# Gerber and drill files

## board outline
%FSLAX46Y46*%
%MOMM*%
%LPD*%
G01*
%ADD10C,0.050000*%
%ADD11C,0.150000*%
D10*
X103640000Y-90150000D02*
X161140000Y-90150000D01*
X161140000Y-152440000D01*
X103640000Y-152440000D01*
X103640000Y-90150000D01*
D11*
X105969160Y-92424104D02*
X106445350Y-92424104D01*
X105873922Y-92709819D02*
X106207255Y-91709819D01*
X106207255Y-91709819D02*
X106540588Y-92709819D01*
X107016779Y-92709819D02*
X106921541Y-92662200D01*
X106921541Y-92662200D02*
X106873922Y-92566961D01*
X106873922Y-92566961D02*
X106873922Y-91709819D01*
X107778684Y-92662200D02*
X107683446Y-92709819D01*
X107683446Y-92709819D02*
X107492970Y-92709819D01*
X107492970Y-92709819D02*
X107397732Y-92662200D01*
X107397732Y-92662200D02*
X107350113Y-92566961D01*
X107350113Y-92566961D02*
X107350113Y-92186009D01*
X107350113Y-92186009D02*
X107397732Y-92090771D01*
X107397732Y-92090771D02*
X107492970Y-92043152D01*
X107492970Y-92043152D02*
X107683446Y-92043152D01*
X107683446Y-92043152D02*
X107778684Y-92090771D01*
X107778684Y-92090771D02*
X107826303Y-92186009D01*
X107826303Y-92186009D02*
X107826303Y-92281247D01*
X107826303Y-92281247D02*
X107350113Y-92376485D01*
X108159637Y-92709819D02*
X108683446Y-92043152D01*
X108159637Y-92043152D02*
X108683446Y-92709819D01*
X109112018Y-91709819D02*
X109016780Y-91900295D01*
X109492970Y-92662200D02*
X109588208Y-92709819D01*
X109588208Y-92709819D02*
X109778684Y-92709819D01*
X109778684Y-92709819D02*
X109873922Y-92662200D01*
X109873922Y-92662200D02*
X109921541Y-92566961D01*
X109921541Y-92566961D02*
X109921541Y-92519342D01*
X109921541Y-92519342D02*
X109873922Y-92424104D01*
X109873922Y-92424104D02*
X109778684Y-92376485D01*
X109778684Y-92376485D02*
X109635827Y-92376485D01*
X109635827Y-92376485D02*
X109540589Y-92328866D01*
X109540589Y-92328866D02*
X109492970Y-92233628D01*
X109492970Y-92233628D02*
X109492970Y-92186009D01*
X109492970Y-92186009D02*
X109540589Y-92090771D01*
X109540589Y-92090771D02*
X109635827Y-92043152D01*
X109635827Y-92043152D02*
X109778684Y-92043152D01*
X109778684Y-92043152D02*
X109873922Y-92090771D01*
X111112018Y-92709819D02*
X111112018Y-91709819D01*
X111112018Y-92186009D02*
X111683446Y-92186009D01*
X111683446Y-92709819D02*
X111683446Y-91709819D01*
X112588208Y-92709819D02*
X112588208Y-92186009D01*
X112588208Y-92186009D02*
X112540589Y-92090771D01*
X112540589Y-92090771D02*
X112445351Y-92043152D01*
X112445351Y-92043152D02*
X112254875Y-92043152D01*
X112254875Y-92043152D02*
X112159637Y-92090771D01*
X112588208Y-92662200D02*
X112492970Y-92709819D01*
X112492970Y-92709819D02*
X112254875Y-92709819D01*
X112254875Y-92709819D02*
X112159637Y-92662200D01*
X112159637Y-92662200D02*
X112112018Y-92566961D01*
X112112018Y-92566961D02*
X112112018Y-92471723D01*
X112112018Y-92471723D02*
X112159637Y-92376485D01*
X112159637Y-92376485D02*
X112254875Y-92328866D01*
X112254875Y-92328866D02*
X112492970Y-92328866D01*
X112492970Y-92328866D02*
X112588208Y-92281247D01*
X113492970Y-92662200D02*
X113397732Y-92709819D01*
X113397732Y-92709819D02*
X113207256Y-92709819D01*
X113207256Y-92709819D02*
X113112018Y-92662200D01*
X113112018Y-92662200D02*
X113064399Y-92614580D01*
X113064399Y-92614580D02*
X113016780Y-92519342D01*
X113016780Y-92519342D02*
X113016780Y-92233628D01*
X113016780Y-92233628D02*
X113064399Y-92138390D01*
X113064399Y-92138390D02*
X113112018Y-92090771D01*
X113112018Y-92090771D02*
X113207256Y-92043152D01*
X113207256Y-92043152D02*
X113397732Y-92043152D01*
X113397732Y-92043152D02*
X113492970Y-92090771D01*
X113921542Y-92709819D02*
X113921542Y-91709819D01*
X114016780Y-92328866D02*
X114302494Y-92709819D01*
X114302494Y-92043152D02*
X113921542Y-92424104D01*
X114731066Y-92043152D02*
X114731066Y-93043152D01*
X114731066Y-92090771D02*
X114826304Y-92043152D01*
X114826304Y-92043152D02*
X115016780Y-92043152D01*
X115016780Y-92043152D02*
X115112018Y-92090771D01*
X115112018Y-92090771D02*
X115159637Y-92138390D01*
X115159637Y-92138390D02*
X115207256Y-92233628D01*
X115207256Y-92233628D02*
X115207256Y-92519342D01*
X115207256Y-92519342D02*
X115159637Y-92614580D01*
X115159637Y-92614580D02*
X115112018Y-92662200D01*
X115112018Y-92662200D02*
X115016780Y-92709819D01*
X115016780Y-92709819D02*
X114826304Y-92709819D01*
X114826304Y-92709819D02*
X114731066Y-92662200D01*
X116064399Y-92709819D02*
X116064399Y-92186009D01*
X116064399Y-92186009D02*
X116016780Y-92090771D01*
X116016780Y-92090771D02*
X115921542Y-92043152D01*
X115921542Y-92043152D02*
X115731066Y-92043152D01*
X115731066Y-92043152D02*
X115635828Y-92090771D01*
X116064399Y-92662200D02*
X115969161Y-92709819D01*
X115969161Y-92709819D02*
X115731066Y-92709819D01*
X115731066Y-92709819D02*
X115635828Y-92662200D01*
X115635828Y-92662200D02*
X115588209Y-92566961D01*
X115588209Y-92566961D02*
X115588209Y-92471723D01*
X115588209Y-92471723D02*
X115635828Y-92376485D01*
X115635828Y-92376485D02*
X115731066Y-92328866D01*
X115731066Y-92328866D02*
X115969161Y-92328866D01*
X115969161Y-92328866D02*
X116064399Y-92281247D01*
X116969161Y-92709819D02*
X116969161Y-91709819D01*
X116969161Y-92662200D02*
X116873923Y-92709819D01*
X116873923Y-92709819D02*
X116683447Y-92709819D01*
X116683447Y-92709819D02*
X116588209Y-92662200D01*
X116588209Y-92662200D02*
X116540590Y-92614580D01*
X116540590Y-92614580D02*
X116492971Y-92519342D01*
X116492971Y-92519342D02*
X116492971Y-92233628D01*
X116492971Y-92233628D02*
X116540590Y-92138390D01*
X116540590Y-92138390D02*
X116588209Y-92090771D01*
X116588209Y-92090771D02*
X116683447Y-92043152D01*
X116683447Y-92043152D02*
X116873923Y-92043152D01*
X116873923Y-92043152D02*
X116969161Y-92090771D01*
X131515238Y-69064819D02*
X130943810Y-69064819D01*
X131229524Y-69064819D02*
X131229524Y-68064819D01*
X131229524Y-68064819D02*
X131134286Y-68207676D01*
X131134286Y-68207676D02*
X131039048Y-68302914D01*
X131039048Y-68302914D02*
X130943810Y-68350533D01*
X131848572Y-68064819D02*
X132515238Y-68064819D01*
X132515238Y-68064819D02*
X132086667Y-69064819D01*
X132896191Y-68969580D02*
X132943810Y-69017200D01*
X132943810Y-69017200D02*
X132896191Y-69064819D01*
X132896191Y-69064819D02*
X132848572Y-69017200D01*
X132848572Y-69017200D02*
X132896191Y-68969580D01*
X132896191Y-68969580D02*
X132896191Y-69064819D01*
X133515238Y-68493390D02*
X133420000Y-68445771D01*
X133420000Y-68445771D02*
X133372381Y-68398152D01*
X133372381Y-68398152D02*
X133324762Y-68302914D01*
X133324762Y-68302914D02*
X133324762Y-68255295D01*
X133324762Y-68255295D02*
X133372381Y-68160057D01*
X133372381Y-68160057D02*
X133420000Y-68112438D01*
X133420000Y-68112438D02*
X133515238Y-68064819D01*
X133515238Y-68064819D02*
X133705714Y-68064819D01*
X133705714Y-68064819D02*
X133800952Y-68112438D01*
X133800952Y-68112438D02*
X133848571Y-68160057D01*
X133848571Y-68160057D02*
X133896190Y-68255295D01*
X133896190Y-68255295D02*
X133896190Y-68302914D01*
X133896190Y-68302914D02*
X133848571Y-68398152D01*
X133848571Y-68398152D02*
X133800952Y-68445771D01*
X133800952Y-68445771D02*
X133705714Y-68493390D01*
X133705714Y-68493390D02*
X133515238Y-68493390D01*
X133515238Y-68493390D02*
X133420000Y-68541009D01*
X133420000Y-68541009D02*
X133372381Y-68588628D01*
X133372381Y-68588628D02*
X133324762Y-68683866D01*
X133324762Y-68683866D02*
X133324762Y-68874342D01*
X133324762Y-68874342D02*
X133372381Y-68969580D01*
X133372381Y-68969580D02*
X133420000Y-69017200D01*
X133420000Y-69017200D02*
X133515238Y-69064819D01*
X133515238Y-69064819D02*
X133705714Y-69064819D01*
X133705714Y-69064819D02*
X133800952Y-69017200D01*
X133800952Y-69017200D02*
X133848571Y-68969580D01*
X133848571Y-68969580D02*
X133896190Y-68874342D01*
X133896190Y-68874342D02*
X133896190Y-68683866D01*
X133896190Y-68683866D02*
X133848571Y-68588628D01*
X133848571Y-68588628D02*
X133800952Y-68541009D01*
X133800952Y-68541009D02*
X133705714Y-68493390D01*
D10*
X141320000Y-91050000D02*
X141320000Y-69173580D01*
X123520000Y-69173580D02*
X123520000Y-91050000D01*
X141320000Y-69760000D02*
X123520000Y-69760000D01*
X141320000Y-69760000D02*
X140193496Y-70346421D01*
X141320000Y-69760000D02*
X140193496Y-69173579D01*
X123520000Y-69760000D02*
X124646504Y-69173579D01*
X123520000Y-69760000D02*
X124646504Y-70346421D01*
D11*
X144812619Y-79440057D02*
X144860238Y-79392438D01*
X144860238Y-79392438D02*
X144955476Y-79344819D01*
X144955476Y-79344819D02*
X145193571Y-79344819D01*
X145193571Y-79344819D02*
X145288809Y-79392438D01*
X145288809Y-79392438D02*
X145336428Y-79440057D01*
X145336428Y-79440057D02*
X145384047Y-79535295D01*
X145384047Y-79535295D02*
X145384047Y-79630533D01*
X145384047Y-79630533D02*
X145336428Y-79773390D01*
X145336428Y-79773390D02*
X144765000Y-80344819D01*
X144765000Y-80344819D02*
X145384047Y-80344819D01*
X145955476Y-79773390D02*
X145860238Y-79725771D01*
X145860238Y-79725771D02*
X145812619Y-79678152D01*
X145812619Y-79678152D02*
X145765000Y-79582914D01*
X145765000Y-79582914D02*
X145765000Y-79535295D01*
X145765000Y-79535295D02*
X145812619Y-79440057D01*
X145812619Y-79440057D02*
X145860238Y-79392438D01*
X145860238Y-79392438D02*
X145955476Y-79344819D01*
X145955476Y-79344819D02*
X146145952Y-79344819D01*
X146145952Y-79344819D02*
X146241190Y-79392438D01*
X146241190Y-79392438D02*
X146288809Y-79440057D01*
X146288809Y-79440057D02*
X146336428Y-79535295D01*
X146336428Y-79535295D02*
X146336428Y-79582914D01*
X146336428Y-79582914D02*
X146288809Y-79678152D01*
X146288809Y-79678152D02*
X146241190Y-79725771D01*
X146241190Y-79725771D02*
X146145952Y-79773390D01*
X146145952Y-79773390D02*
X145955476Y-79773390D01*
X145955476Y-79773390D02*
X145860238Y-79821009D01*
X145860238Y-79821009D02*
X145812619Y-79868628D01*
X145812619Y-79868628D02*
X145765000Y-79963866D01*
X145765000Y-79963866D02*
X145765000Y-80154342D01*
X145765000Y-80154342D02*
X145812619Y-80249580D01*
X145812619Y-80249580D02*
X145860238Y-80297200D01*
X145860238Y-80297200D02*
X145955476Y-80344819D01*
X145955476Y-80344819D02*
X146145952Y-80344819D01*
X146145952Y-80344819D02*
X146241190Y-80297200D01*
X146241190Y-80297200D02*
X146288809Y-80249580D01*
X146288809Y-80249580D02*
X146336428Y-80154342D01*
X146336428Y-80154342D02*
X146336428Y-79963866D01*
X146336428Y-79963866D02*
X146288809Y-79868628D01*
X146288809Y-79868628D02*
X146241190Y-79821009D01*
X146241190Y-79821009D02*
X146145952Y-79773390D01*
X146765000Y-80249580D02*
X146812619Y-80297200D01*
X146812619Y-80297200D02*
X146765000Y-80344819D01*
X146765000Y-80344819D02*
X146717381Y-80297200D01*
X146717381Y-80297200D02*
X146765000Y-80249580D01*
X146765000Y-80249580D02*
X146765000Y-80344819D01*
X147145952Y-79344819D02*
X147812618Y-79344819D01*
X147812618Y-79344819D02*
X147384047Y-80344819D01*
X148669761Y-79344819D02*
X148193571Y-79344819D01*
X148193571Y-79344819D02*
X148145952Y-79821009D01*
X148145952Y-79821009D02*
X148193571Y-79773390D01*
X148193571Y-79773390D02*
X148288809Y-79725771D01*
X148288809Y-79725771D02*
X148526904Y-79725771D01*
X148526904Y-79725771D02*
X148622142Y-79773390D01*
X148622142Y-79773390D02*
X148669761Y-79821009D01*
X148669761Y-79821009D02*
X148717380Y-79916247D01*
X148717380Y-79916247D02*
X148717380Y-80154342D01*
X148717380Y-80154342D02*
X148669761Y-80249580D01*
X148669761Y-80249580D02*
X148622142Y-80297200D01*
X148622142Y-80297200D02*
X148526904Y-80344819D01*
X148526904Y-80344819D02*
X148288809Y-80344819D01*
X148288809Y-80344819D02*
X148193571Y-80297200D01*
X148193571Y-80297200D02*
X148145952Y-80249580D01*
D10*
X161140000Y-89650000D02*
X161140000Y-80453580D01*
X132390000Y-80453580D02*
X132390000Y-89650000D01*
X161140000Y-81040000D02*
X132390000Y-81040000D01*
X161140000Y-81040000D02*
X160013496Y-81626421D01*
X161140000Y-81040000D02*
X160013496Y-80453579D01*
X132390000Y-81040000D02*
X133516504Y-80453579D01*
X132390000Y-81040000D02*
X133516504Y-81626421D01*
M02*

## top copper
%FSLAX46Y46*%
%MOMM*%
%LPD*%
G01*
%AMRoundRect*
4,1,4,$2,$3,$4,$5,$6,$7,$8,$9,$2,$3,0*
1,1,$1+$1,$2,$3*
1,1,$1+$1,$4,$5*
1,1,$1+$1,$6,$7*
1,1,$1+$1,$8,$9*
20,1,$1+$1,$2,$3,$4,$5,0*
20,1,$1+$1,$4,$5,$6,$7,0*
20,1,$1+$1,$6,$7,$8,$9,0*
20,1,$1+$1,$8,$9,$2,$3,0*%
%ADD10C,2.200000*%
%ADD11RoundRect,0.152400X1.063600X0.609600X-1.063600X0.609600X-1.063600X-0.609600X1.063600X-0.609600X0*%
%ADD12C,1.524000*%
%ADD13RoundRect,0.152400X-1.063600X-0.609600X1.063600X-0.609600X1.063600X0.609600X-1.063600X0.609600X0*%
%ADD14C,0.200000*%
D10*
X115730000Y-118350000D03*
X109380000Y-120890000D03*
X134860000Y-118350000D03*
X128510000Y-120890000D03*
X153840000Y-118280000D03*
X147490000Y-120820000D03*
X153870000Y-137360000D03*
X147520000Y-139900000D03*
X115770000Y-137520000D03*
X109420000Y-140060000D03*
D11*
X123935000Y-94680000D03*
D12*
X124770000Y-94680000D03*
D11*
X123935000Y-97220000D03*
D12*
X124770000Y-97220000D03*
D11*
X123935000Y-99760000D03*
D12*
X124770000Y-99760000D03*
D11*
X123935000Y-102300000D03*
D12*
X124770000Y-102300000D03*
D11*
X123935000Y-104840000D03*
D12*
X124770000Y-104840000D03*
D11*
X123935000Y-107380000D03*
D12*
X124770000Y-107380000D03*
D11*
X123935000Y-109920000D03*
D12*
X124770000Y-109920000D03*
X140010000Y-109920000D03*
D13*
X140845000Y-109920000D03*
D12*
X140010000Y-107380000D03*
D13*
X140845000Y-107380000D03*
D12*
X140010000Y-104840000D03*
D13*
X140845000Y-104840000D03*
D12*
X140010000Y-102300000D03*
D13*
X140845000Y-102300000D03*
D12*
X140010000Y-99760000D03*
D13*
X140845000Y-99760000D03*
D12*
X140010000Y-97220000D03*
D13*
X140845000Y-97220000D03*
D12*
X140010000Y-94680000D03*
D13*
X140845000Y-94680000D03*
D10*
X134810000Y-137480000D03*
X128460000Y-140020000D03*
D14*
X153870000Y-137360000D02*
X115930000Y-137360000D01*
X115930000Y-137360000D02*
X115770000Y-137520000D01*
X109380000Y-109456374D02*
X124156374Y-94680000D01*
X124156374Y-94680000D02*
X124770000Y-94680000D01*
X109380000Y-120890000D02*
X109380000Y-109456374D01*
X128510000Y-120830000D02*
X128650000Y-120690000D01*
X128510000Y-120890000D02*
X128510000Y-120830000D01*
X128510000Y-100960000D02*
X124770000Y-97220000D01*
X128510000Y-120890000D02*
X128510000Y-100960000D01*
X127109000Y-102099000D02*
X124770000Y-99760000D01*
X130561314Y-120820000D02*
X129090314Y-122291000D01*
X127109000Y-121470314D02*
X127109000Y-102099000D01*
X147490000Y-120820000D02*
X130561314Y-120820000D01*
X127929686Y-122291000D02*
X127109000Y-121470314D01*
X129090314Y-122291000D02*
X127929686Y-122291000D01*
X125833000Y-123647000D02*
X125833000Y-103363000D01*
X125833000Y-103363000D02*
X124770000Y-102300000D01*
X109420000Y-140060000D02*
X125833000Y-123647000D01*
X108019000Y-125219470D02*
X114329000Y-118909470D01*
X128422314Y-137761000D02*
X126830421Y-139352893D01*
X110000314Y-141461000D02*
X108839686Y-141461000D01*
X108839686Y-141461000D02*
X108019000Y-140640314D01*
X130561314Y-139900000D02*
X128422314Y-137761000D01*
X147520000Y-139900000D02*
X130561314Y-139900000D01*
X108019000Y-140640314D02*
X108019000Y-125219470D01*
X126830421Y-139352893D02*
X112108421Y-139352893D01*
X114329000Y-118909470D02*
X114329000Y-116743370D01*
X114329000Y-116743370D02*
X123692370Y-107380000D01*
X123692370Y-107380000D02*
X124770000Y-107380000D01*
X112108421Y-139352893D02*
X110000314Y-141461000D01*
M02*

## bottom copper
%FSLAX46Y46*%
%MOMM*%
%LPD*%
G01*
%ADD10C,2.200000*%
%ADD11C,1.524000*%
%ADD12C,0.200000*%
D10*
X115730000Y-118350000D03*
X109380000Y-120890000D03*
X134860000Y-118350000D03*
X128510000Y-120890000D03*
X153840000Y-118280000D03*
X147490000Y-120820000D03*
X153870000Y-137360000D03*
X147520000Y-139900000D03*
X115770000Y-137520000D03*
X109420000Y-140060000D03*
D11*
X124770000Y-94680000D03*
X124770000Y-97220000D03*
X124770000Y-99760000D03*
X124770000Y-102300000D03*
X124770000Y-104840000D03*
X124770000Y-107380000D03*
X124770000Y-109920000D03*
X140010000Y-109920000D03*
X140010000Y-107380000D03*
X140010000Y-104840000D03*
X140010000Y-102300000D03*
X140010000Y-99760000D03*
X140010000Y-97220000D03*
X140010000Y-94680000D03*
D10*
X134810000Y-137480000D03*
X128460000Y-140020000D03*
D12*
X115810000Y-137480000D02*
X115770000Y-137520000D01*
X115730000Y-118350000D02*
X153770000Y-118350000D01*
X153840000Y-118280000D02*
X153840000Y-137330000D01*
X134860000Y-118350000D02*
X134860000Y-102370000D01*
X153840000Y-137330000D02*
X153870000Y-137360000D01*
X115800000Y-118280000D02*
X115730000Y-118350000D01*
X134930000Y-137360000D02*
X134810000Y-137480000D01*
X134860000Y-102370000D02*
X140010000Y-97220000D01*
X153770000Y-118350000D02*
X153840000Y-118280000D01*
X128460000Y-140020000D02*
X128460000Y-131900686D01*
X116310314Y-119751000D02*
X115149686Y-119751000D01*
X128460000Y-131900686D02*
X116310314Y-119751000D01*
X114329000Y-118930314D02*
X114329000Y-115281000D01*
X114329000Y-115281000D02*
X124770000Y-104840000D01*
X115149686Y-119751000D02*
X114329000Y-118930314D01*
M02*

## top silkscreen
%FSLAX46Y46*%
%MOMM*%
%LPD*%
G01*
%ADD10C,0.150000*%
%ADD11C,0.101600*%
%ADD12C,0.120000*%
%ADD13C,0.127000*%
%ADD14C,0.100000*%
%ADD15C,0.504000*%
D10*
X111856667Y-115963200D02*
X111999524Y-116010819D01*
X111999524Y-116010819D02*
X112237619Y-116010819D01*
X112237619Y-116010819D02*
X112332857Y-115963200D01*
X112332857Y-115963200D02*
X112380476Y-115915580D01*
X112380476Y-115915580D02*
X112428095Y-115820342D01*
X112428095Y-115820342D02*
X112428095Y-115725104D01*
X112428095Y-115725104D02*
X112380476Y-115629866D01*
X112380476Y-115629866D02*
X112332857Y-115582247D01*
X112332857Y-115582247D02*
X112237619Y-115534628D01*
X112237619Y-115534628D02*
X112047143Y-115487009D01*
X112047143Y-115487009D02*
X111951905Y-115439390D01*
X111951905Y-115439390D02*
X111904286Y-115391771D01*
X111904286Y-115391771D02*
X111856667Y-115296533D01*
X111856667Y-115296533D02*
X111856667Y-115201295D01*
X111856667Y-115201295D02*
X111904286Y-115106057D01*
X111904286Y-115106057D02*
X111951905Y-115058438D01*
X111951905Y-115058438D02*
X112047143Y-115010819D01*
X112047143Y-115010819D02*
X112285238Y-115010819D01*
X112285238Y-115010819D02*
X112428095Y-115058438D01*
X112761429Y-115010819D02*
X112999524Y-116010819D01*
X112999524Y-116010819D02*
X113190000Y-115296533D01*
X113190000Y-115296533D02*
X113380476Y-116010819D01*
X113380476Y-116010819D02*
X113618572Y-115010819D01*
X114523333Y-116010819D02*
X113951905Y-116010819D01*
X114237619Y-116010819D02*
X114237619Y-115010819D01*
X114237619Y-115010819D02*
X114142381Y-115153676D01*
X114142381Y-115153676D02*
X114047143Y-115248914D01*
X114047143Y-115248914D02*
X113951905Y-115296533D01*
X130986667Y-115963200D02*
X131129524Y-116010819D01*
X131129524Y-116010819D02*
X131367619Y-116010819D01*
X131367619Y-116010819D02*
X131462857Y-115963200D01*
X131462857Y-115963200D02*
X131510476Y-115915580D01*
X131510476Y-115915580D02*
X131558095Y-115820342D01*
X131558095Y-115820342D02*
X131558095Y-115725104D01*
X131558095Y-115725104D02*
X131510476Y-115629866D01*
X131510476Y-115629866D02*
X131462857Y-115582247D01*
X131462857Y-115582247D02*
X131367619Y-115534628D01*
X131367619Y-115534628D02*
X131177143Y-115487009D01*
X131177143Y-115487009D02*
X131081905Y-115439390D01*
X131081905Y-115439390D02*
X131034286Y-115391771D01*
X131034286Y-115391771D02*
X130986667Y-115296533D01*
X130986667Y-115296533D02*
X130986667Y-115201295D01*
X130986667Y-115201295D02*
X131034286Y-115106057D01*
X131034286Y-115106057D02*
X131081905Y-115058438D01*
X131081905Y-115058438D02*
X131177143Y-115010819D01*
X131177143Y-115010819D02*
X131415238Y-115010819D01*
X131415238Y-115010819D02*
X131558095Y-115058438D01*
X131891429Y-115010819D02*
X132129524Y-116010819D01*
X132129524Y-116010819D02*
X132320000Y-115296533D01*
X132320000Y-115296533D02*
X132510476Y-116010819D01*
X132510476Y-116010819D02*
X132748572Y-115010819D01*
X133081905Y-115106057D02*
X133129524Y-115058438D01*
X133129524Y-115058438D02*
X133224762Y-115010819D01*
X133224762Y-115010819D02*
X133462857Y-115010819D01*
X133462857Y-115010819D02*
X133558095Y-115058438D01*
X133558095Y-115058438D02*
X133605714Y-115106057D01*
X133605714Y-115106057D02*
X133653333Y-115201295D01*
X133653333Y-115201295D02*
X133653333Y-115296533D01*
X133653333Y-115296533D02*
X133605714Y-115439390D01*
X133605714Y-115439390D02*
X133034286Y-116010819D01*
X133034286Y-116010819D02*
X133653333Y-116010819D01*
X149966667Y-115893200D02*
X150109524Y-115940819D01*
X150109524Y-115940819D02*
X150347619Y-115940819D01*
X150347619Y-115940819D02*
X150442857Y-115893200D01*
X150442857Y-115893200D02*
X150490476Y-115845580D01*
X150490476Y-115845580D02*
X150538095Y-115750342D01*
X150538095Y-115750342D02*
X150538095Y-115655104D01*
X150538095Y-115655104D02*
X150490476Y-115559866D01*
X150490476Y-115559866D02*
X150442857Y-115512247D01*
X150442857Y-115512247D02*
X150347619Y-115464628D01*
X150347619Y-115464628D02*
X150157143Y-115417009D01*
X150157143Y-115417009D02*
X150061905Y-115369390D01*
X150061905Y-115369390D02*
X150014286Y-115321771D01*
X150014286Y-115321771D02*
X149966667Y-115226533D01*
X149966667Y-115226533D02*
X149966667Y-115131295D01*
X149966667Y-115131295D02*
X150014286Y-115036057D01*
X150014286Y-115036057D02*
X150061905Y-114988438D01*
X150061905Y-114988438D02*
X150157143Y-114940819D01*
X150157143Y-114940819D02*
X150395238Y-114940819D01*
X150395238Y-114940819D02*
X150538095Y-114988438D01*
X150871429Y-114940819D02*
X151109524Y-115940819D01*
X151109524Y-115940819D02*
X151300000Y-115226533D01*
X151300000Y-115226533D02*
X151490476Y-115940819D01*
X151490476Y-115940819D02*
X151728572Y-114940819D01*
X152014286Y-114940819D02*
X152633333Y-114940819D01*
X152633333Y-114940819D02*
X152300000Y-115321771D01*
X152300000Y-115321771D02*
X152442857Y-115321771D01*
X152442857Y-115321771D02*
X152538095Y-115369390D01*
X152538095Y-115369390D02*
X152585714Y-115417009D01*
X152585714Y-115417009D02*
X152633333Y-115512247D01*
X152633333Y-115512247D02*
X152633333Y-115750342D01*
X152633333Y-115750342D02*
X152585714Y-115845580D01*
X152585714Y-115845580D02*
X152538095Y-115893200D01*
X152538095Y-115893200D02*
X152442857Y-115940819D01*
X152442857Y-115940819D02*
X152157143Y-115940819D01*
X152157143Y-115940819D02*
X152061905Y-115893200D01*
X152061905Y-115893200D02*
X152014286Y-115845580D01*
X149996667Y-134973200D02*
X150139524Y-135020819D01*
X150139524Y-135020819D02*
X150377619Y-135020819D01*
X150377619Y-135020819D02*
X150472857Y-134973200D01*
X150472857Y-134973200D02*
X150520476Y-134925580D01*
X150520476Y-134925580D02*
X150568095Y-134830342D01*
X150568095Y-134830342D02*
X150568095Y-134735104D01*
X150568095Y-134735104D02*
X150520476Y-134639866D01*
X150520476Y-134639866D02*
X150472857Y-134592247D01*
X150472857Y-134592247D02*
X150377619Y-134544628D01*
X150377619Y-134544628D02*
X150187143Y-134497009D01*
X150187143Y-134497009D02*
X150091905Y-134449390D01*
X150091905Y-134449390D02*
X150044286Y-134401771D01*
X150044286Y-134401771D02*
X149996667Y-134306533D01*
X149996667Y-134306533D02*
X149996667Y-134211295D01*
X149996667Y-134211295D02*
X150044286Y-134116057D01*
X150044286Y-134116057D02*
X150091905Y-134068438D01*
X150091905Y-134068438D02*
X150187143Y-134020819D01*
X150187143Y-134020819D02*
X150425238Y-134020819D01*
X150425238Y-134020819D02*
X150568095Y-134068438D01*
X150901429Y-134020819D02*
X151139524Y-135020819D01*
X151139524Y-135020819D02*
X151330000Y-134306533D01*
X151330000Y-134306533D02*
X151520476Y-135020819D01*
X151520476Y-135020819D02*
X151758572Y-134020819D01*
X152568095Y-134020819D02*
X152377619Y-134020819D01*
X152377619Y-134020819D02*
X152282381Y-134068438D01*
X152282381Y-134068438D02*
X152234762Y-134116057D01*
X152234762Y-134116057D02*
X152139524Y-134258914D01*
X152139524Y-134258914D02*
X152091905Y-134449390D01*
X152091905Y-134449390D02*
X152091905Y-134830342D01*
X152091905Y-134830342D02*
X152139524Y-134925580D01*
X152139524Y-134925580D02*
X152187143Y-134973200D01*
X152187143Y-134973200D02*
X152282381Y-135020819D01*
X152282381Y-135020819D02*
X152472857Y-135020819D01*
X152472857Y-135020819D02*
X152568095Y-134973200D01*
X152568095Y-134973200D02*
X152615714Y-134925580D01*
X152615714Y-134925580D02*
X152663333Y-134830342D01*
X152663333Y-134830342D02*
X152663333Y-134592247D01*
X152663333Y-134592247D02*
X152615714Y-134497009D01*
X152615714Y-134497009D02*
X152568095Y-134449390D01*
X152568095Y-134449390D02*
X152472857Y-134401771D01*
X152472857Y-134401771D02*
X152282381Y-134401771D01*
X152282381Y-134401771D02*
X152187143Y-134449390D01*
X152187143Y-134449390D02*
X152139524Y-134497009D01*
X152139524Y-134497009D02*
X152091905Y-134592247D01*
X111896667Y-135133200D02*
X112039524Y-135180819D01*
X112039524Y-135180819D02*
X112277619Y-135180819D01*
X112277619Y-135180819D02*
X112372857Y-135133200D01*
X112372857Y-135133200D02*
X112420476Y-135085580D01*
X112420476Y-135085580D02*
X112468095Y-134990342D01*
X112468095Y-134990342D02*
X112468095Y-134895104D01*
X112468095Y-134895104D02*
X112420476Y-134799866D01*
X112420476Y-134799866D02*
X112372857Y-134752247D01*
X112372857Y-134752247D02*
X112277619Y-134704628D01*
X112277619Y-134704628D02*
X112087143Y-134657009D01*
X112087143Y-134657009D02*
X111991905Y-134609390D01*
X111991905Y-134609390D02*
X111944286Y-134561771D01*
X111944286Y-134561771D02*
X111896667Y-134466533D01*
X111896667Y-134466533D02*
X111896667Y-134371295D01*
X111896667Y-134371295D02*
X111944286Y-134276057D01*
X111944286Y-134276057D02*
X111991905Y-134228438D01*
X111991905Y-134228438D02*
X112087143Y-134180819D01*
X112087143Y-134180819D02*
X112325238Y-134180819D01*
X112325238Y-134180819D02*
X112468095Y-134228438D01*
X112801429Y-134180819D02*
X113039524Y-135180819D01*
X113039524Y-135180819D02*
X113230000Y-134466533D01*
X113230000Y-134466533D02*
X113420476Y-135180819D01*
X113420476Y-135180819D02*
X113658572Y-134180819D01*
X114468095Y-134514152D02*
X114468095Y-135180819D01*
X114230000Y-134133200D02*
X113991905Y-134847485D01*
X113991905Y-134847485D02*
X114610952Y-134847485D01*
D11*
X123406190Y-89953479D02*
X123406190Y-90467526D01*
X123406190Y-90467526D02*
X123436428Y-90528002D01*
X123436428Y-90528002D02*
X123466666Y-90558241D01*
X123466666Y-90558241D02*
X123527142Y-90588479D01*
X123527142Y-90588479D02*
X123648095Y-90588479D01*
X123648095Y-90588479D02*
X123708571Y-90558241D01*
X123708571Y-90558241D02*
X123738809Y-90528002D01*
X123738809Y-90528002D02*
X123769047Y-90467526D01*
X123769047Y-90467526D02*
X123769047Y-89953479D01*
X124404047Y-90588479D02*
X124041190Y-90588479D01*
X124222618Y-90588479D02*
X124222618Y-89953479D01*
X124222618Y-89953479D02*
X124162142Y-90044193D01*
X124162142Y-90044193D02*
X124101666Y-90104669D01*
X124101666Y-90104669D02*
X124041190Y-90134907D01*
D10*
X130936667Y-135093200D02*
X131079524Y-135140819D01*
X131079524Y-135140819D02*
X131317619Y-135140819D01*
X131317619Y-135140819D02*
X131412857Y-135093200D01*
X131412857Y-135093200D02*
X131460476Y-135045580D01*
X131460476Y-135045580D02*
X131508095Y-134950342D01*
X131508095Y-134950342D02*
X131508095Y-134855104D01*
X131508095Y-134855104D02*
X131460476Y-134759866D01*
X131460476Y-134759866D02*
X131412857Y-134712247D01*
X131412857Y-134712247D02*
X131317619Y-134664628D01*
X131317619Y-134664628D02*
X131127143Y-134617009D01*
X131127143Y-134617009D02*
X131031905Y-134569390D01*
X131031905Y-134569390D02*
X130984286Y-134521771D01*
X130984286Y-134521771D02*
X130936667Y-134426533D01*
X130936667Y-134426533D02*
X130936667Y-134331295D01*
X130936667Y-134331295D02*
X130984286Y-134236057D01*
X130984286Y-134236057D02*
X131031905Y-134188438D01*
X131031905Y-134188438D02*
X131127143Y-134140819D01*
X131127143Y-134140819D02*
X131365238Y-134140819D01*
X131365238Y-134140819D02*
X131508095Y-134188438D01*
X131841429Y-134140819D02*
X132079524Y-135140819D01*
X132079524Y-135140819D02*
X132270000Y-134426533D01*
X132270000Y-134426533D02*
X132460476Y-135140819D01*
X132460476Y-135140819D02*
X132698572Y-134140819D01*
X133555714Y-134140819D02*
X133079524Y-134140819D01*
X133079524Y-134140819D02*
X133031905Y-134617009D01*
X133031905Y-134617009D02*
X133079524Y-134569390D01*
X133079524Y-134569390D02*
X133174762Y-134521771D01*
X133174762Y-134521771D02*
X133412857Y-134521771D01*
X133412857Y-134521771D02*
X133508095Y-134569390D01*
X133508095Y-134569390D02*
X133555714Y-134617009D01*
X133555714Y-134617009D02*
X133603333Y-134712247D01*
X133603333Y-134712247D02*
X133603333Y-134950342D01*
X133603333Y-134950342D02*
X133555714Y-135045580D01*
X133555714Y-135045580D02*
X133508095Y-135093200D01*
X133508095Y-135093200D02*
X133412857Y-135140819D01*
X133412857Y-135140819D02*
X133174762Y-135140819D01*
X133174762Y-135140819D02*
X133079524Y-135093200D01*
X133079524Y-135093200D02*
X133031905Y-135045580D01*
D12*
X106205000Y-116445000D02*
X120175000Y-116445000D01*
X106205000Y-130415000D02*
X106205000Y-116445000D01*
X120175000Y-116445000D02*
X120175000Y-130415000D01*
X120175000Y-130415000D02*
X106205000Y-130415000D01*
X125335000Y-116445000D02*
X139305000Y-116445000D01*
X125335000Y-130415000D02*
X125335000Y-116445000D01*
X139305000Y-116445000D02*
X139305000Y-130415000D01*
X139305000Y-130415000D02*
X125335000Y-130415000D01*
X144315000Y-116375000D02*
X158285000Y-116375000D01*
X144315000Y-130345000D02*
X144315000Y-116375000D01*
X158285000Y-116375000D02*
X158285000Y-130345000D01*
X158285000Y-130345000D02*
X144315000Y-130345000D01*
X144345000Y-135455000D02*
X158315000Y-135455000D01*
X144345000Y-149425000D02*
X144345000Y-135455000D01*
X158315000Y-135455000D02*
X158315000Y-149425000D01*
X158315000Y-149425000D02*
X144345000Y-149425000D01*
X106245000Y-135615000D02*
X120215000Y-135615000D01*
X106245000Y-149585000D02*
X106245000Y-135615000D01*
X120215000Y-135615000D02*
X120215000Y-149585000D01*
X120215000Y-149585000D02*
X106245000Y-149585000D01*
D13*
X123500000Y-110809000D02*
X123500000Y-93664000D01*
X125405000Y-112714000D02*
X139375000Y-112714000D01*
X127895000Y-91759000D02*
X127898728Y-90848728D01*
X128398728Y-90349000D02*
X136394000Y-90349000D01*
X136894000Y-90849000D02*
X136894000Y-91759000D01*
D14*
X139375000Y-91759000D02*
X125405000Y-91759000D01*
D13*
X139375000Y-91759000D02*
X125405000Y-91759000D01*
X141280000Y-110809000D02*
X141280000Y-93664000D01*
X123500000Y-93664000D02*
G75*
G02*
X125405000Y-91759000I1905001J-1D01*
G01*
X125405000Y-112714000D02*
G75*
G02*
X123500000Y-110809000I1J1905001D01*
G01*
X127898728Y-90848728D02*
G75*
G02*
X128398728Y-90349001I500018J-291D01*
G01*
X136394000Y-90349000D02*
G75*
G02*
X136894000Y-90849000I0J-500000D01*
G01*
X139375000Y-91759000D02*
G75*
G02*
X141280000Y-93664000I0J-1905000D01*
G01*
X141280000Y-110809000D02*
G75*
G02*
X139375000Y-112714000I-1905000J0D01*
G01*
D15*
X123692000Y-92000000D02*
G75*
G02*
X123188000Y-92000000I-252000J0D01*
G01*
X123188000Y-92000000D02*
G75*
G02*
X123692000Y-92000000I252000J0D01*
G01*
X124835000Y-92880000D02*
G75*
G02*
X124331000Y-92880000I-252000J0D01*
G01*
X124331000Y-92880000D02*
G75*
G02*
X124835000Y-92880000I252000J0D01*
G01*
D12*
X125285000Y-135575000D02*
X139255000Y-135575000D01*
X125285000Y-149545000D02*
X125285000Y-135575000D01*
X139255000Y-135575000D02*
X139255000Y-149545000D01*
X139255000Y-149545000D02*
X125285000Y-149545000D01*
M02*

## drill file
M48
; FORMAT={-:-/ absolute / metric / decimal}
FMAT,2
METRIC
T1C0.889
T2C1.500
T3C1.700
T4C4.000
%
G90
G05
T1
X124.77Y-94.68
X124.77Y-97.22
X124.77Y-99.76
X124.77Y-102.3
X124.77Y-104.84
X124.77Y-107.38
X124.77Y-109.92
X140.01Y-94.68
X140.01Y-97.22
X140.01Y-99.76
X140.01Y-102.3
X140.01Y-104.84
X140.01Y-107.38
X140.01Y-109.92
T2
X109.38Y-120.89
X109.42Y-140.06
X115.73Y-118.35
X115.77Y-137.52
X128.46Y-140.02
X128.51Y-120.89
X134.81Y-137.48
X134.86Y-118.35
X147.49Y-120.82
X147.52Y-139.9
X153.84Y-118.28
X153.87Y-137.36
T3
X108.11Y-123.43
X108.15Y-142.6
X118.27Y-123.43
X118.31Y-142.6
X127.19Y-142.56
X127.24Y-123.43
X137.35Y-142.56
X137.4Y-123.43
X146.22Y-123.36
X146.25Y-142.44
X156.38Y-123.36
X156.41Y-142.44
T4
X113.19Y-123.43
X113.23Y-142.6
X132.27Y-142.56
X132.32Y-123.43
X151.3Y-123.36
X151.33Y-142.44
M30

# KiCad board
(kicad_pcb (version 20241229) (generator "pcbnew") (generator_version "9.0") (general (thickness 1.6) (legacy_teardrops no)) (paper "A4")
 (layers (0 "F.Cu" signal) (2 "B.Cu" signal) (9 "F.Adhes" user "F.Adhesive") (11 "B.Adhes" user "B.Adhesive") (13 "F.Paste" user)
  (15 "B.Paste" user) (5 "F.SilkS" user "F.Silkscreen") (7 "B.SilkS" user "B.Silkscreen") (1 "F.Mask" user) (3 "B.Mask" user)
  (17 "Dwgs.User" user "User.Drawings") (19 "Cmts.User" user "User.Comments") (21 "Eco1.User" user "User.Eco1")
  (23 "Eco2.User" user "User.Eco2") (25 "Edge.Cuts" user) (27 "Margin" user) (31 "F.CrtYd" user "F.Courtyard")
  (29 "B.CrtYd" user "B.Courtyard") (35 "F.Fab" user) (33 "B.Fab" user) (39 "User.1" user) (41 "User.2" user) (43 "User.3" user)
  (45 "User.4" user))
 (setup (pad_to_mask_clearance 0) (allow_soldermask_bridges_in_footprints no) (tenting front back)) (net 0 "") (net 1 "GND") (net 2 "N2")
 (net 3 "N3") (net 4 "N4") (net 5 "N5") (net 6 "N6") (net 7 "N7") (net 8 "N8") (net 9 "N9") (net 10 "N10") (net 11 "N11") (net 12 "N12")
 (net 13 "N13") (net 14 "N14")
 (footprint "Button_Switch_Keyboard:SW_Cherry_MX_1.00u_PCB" (layer "F.Cu") (at 115.73 118.35)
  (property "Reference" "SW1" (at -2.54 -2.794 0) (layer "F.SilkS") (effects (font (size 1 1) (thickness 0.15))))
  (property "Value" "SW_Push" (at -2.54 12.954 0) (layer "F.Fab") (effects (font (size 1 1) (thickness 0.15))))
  (fp_line (start -9.525 -1.905) (end 4.445 -1.905) (stroke (width 0.12) (type solid)) (layer "F.SilkS"))
  (fp_line (start -9.525 12.065) (end -9.525 -1.905) (stroke (width 0.12) (type solid)) (layer "F.SilkS"))
  (fp_line (start 4.445 -1.905) (end 4.445 12.065) (stroke (width 0.12) (type solid)) (layer "F.SilkS"))
  (fp_line (start 4.445 12.065) (end -9.525 12.065) (stroke (width 0.12) (type solid)) (layer "F.SilkS"))
  (pad "" np_thru_hole circle (at -7.62 5.08) (size 1.7 1.7) (drill 1.7) (layers "*.Cu" "*.Mask"))
  (pad "" np_thru_hole circle (at -2.54 5.08) (size 4 4) (drill 4) (layers "*.Cu" "*.Mask"))
  (pad "" np_thru_hole circle (at 2.54 5.08) (size 1.7 1.7) (drill 1.7) (layers "*.Cu" "*.Mask"))
  (pad "1" thru_hole circle (at 0 0) (size 2.2 2.2) (drill 1.5) (layers "*.Cu" "*.Mask") (remove_unused_layers no) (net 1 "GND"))
  (pad "2" thru_hole circle (at -6.35 2.54) (size 2.2 2.2) (drill 1.5) (layers "*.Cu" "*.Mask") (remove_unused_layers no) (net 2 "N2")))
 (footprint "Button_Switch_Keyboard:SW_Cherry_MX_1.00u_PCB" (layer "F.Cu") (at 134.86 118.35)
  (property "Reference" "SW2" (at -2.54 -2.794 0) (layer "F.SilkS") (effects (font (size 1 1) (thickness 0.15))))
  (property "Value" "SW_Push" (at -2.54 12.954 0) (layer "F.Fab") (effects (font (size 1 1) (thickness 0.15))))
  (fp_line (start -9.525 -1.905) (end 4.445 -1.905) (stroke (width 0.12) (type solid)) (layer "F.SilkS"))
  (fp_line (start -9.525 12.065) (end -9.525 -1.905) (stroke (width 0.12) (type solid)) (layer "F.SilkS"))
  (fp_line (start 4.445 -1.905) (end 4.445 12.065) (stroke (width 0.12) (type solid)) (layer "F.SilkS"))
  (fp_line (start 4.445 12.065) (end -9.525 12.065) (stroke (width 0.12) (type solid)) (layer "F.SilkS"))
  (pad "" np_thru_hole circle (at -7.62 5.08) (size 1.7 1.7) (drill 1.7) (layers "*.Cu" "*.Mask"))
  (pad "" np_thru_hole circle (at -2.54 5.08) (size 4 4) (drill 4) (layers "*.Cu" "*.Mask"))
  (pad "" np_thru_hole circle (at 2.54 5.08) (size 1.7 1.7) (drill 1.7) (layers "*.Cu" "*.Mask"))
  (pad "1" thru_hole circle (at 0 0) (size 2.2 2.2) (drill 1.5) (layers "*.Cu" "*.Mask") (remove_unused_layers no) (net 1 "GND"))
  (pad "2" thru_hole circle (at -6.35 2.54) (size 2.2 2.2) (drill 1.5) (layers "*.Cu" "*.Mask") (remove_unused_layers no) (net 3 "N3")))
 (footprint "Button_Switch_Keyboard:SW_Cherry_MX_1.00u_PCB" (layer "F.Cu") (at 153.84 118.28)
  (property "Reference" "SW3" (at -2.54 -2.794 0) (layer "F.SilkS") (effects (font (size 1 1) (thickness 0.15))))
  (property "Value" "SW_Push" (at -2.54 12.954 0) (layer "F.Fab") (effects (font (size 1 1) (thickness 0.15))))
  (fp_line (start -9.525 -1.905) (end 4.445 -1.905) (stroke (width 0.12) (type solid)) (layer "F.SilkS"))
  (fp_line (start -9.525 12.065) (end -9.525 -1.905) (stroke (width 0.12) (type solid)) (layer "F.SilkS"))
  (fp_line (start 4.445 -1.905) (end 4.445 12.065) (stroke (width 0.12) (type solid)) (layer "F.SilkS"))
  (fp_line (start 4.445 12.065) (end -9.525 12.065) (stroke (width 0.12) (type solid)) (layer "F.SilkS"))
  (pad "" np_thru_hole circle (at -7.62 5.08) (size 1.7 1.7) (drill 1.7) (layers "*.Cu" "*.Mask"))
  (pad "" np_thru_hole circle (at -2.54 5.08) (size 4 4) (drill 4) (layers "*.Cu" "*.Mask"))
  (pad "" np_thru_hole circle (at 2.54 5.08) (size 1.7 1.7) (drill 1.7) (layers "*.Cu" "*.Mask"))
  (pad "1" thru_hole circle (at 0 0) (size 2.2 2.2) (drill 1.5) (layers "*.Cu" "*.Mask") (remove_unused_layers no) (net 1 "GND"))
  (pad "2" thru_hole circle (at -6.35 2.54) (size 2.2 2.2) (drill 1.5) (layers "*.Cu" "*.Mask") (remove_unused_layers no) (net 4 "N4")))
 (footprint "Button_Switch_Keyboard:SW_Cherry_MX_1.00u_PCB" (layer "F.Cu") (at 153.87 137.36)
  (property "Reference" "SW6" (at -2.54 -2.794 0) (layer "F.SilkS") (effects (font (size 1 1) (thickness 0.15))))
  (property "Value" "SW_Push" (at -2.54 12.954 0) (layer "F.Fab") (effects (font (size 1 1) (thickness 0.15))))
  (fp_line (start -9.525 -1.905) (end 4.445 -1.905) (stroke (width 0.12) (type solid)) (layer "F.SilkS"))
  (fp_line (start -9.525 12.065) (end -9.525 -1.905) (stroke (width 0.12) (type solid)) (layer "F.SilkS"))
  (fp_line (start 4.445 -1.905) (end 4.445 12.065) (stroke (width 0.12) (type solid)) (layer "F.SilkS"))
  (fp_line (start 4.445 12.065) (end -9.525 12.065) (stroke (width 0.12) (type solid)) (layer "F.SilkS"))
  (pad "" np_thru_hole circle (at -7.62 5.08) (size 1.7 1.7) (drill 1.7) (layers "*.Cu" "*.Mask"))
  (pad "" np_thru_hole circle (at -2.54 5.08) (size 4 4) (drill 4) (layers "*.Cu" "*.Mask"))
  (pad "" np_thru_hole circle (at 2.54 5.08) (size 1.7 1.7) (drill 1.7) (layers "*.Cu" "*.Mask"))
  (pad "1" thru_hole circle (at 0 0) (size 2.2 2.2) (drill 1.5) (layers "*.Cu" "*.Mask") (remove_unused_layers no) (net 1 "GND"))
  (pad "2" thru_hole circle (at -6.35 2.54) (size 2.2 2.2) (drill 1.5) (layers "*.Cu" "*.Mask") (remove_unused_layers no) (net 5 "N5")))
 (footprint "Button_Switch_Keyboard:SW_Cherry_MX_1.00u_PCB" (layer "F.Cu") (at 115.77 137.52)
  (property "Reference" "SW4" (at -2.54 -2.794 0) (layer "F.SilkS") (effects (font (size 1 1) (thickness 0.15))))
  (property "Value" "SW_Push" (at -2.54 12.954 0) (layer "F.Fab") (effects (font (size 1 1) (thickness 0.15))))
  (fp_line (start -9.525 -1.905) (end 4.445 -1.905) (stroke (width 0.12) (type solid)) (layer "F.SilkS"))
  (fp_line (start -9.525 12.065) (end -9.525 -1.905) (stroke (width 0.12) (type solid)) (layer "F.SilkS"))
  (fp_line (start 4.445 -1.905) (end 4.445 12.065) (stroke (width 0.12) (type solid)) (layer "F.SilkS"))
  (fp_line (start 4.445 12.065) (end -9.525 12.065) (stroke (width 0.12) (type solid)) (layer "F.SilkS"))
  (pad "" np_thru_hole circle (at -7.62 5.08) (size 1.7 1.7) (drill 1.7) (layers "*.Cu" "*.Mask"))
  (pad "" np_thru_hole circle (at -2.54 5.08) (size 4 4) (drill 4) (layers "*.Cu" "*.Mask"))
  (pad "" np_thru_hole circle (at 2.54 5.08) (size 1.7 1.7) (drill 1.7) (layers "*.Cu" "*.Mask"))
  (pad "1" thru_hole circle (at 0 0) (size 2.2 2.2) (drill 1.5) (layers "*.Cu" "*.Mask") (remove_unused_layers no) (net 1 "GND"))
  (pad "2" thru_hole circle (at -6.35 2.54) (size 2.2 2.2) (drill 1.5) (layers "*.Cu" "*.Mask") (remove_unused_layers no) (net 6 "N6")))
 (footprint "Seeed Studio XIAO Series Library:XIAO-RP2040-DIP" (layer "F.Cu") (at 132.39 102.3)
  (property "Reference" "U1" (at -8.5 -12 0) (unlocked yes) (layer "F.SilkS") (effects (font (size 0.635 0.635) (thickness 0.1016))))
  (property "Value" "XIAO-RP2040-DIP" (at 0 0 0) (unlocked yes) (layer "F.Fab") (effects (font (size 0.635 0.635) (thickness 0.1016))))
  (fp_line (start -8.89 8.509) (end -8.89 -8.636) (stroke (width 0.127) (type solid)) (layer "F.SilkS"))
  (fp_line (start -6.985 10.414) (end 6.985 10.414) (stroke (width 0.127) (type solid)) (layer "F.SilkS"))
  (fp_line (start -4.495 -10.541) (end -4.491272 -11.451272) (stroke (width 0.127) (type solid)) (layer "F.SilkS"))
  (fp_line (start -3.991272 -11.951) (end 4.004 -11.951) (stroke (width 0.127) (type solid)) (layer "F.SilkS"))
  (fp_line (start 4.504 -11.451) (end 4.504 -10.541) (stroke (width 0.127) (type solid)) (layer "F.SilkS"))
  (fp_line (start 6.985 -10.541) (end -6.985 -10.541) (stroke (width 0.1) (type solid)) (layer "F.SilkS"))
  (fp_line (start 6.985 -10.541) (end -6.985 -10.541) (stroke (width 0.127) (type solid)) (layer "F.SilkS"))
  (fp_line (start 8.89 8.509) (end 8.89 -8.636) (stroke (width 0.127) (type solid)) (layer "F.SilkS"))
  (fp_arc (start -8.89 -8.636) (mid -8.332038 -9.983038) (end -6.985 -10.541) (stroke (width 0.127) (type solid)) (layer "F.SilkS"))
  (fp_arc (start -6.985 10.414) (mid -8.332038 9.856038) (end -8.89 8.509) (stroke (width 0.127) (type solid)) (layer "F.SilkS"))
  (fp_arc (start -4.491272 -11.451272) (mid -4.344728 -11.80464) (end -3.991272 -11.951) (stroke (width 0.127) (type default))
   (layer "F.SilkS"))
  (fp_arc (start 4.004 -11.951) (mid 4.357553 -11.804553) (end 4.504 -11.451) (stroke (width 0.127) (type default)) (layer "F.SilkS"))
  (fp_arc (start 6.985 -10.541) (mid 8.332038 -9.983038) (end 8.89 -8.636) (stroke (width 0.127) (type solid)) (layer "F.SilkS"))
  (fp_arc (start 8.89 8.509) (mid 8.332038 9.856038) (end 6.985 10.414) (stroke (width 0.127) (type solid)) (layer "F.SilkS"))
  (fp_circle (center -8.95 -10.3) (end -8.95 -10.554) (stroke (width 0.5) (type solid)) (fill yes) (layer "F.SilkS"))
  (fp_circle (center -7.807 -9.42) (end -7.807 -9.674) (stroke (width 0.5) (type solid)) (fill yes) (layer "F.SilkS"))
  (pad "1" smd roundrect (at -8.455 -7.62 180) (size 2.432 1.524) (layers "F.Cu" "F.Mask") (roundrect_rratio 0.1) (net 2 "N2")
   (thermal_bridge_angle 45))
  (pad "1" thru_hole circle (at -7.62 -7.62 180) (size 1.524 1.524) (drill 0.889) (layers "*.Cu" "*.Mask") (remove_unused_layers no)
   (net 2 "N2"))
  (pad "2" smd roundrect (at -8.455 -5.08 180) (size 2.432 1.524) (layers "F.Cu" "F.Mask") (roundrect_rratio 0.1) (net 3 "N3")
   (thermal_bridge_angle 45))
  (pad "2" thru_hole circle (at -7.62 -5.08 180) (size 1.524 1.524) (drill 0.889) (layers "*.Cu" "*.Mask") (remove_unused_layers no)
   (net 3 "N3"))
  (pad "3" smd roundrect (at -8.455 -2.54 180) (size 2.432 1.524) (layers "F.Cu" "F.Mask") (roundrect_rratio 0.1) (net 4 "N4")
   (thermal_bridge_angle 45))
  (pad "3" thru_hole circle (at -7.62 -2.54 180) (size 1.524 1.524) (drill 0.889) (layers "*.Cu" "*.Mask") (remove_unused_layers no)
   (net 4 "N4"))
  (pad "4" smd roundrect (at -8.455 0 180) (size 2.432 1.524) (layers "F.Cu" "F.Mask") (roundrect_rratio 0.1) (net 6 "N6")
   (thermal_bridge_angle 45))
  (pad "4" thru_hole circle (at -7.62 0 180) (size 1.524 1.524) (drill 0.889) (layers "*.Cu" "*.Mask") (remove_unused_layers no)
   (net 6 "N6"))
  (pad "5" smd roundrect (at -8.455 2.54 180) (size 2.432 1.524) (layers "F.Cu" "F.Mask") (roundrect_rratio 0.1) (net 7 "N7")
   (thermal_bridge_angle 45))
  (pad "5" thru_hole circle (at -7.62 2.54 180) (size 1.524 1.524) (drill 0.889) (layers "*.Cu" "*.Mask") (remove_unused_layers no)
   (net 7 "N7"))
  (pad "6" smd roundrect (at -8.455 5.08 180) (size 2.432 1.524) (layers "F.Cu" "F.Mask") (roundrect_rratio 0.1) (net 5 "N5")
   (thermal_bridge_angle 45))
  (pad "6" thru_hole circle (at -7.62 5.08 180) (size 1.524 1.524) (drill 0.889) (layers "*.Cu" "*.Mask") (remove_unused_layers no)
   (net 5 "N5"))
  (pad "7" smd roundrect (at -8.455 7.62 180) (size 2.432 1.524) (layers "F.Cu" "F.Mask") (roundrect_rratio 0.1) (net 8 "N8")
   (thermal_bridge_angle 45))
  (pad "7" thru_hole circle (at -7.62 7.62 180) (size 1.524 1.524) (drill 0.889) (layers "*.Cu" "*.Mask") (remove_unused_layers no)
   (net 8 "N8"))
  (pad "8" thru_hole circle (at 7.62 7.62) (size 1.524 1.524) (drill 0.889) (layers "*.Cu" "*.Mask") (remove_unused_layers no) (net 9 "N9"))
  (pad "8" smd roundrect (at 8.455 7.62) (size 2.432 1.524) (layers "F.Cu" "F.Mask") (roundrect_rratio 0.1) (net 9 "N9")
   (thermal_bridge_angle 45))
  (pad "9" thru_hole circle (at 7.62 5.08) (size 1.524 1.524) (drill 0.889) (layers "*.Cu" "*.Mask") (remove_unused_layers no)
   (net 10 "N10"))
  (pad "9" smd roundrect (at 8.455 5.08) (size 2.432 1.524) (layers "F.Cu" "F.Mask") (roundrect_rratio 0.1) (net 10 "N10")
   (thermal_bridge_angle 45))
  (pad "10" thru_hole circle (at 7.62 2.54) (size 1.524 1.524) (drill 0.889) (layers "*.Cu" "*.Mask") (remove_unused_layers no)
   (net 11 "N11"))
  (pad "10" smd roundrect (at 8.455 2.54) (size 2.432 1.524) (layers "F.Cu" "F.Mask") (roundrect_rratio 0.1) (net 11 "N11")
   (thermal_bridge_angle 45))
  (pad "11" thru_hole circle (at 7.62 0) (size 1.524 1.524) (drill 0.889) (layers "*.Cu" "*.Mask") (remove_unused_layers no) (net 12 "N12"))
  (pad "11" smd roundrect (at 8.455 0) (size 2.432 1.524) (layers "F.Cu" "F.Mask") (roundrect_rratio 0.1) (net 12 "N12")
   (thermal_bridge_angle 45))
  (pad "12" thru_hole circle (at 7.62 -2.54) (size 1.524 1.524) (drill 0.889) (layers "*.Cu" "*.Mask") (remove_unused_layers no)
   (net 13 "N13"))
  (pad "12" smd roundrect (at 8.455 -2.54) (size 2.432 1.524) (layers "F.Cu" "F.Mask") (roundrect_rratio 0.1) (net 13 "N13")
   (thermal_bridge_angle 45))
  (pad "13" thru_hole circle (at 7.62 -5.08) (size 1.524 1.524) (drill 0.889) (layers "*.Cu" "*.Mask") (remove_unused_layers no)
   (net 1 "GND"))
  (pad "13" smd roundrect (at 8.455 -5.08) (size 2.432 1.524) (layers "F.Cu" "F.Mask") (roundrect_rratio 0.1) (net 1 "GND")
   (thermal_bridge_angle 45))
  (pad "14" thru_hole circle (at 7.62 -7.62) (size 1.524 1.524) (drill 0.889) (layers "*.Cu" "*.Mask") (remove_unused_layers no)
   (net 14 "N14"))
  (pad "14" smd roundrect (at 8.455 -7.62) (size 2.432 1.524) (layers "F.Cu" "F.Mask") (roundrect_rratio 0.1) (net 14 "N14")
   (thermal_bridge_angle 45)))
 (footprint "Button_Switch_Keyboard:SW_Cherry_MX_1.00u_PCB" (layer "F.Cu") (at 134.81 137.48)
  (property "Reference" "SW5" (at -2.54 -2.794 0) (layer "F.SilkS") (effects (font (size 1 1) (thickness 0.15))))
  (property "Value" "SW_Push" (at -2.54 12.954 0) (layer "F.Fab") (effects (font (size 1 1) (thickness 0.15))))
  (fp_line (start -9.525 -1.905) (end 4.445 -1.905) (stroke (width 0.12) (type solid)) (layer "F.SilkS"))
  (fp_line (start -9.525 12.065) (end -9.525 -1.905) (stroke (width 0.12) (type solid)) (layer "F.SilkS"))
  (fp_line (start 4.445 -1.905) (end 4.445 12.065) (stroke (width 0.12) (type solid)) (layer "F.SilkS"))
  (fp_line (start 4.445 12.065) (end -9.525 12.065) (stroke (width 0.12) (type solid)) (layer "F.SilkS"))
  (pad "" np_thru_hole circle (at -7.62 5.08) (size 1.7 1.7) (drill 1.7) (layers "*.Cu" "*.Mask"))
  (pad "" np_thru_hole circle (at -2.54 5.08) (size 4 4) (drill 4) (layers "*.Cu" "*.Mask"))
  (pad "" np_thru_hole circle (at 2.54 5.08) (size 1.7 1.7) (drill 1.7) (layers "*.Cu" "*.Mask"))
  (pad "1" thru_hole circle (at 0 0) (size 2.2 2.2) (drill 1.5) (layers "*.Cu" "*.Mask") (remove_unused_layers no) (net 1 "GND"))
  (pad "2" thru_hole circle (at -6.35 2.54) (size 2.2 2.2) (drill 1.5) (layers "*.Cu" "*.Mask") (remove_unused_layers no) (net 7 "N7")))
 (gr_rect (start 103.64 90.15) (end 161.14 152.44) (stroke (width 0.05) (type default)) (fill no) (layer "Edge.Cuts"))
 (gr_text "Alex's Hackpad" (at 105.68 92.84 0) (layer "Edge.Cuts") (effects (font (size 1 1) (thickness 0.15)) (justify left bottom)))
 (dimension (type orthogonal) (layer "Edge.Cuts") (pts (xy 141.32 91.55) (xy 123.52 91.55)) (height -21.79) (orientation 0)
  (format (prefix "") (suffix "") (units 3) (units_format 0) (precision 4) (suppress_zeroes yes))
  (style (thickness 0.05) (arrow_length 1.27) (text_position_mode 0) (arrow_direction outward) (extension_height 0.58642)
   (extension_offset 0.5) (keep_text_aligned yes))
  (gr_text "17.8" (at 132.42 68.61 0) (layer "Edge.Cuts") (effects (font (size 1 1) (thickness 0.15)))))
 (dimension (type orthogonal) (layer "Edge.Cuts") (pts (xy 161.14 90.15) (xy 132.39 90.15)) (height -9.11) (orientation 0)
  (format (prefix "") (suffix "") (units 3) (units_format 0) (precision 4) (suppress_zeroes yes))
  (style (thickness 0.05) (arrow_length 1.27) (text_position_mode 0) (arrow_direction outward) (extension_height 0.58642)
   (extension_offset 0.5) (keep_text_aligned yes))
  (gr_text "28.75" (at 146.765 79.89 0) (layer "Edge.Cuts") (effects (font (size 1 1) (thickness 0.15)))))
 (segment (start 153.87 137.36) (end 115.93 137.36) (width 0.2) (layer "F.Cu") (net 1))
 (segment (start 115.93 137.36) (end 115.77 137.52) (width 0.2) (layer "F.Cu") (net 1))
 (segment (start 115.81 137.48) (end 115.77 137.52) (width 0.2) (layer "B.Cu") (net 1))
 (segment (start 115.73 118.35) (end 153.77 118.35) (width 0.2) (layer "B.Cu") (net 1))
 (segment (start 153.84 118.28) (end 153.84 137.33) (width 0.2) (layer "B.Cu") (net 1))
 (segment (start 134.86 118.35) (end 134.86 102.37) (width 0.2) (layer "B.Cu") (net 1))
 (segment (start 153.84 137.33) (end 153.87 137.36) (width 0.2) (layer "B.Cu") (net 1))
 (segment (start 115.8 118.28) (end 115.73 118.35) (width 0.2) (layer "B.Cu") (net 1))
 (segment (start 134.93 137.36) (end 134.81 137.48) (width 0.2) (layer "B.Cu") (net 1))
 (segment (start 134.86 102.37) (end 140.01 97.22) (width 0.2) (layer "B.Cu") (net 1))
 (segment (start 153.77 118.35) (end 153.84 118.28) (width 0.2) (layer "B.Cu") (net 1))
 (segment (start 109.38 109.456374) (end 124.156374 94.68) (width 0.2) (layer "F.Cu") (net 2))
 (segment (start 124.156374 94.68) (end 124.77 94.68) (width 0.2) (layer "F.Cu") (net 2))
 (segment (start 109.38 120.89) (end 109.38 109.456374) (width 0.2) (layer "F.Cu") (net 2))
 (segment (start 128.51 120.83) (end 128.65 120.69) (width 0.2) (layer "F.Cu") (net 3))
 (segment (start 128.51 120.89) (end 128.51 120.83) (width 0.2) (layer "F.Cu") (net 3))
 (segment (start 128.51 100.96) (end 124.77 97.22) (width 0.2) (layer "F.Cu") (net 3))
 (segment (start 128.51 120.89) (end 128.51 100.96) (width 0.2) (layer "F.Cu") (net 3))
 (segment (start 127.109 102.099) (end 124.77 99.76) (width 0.2) (layer "F.Cu") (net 4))
 (segment (start 130.561314 120.82) (end 129.090314 122.291) (width 0.2) (layer "F.Cu") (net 4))
 (segment (start 127.109 121.470314) (end 127.109 102.099) (width 0.2) (layer "F.Cu") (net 4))
 (segment (start 147.49 120.82) (end 130.561314 120.82) (width 0.2) (layer "F.Cu") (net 4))
 (segment (start 127.929686 122.291) (end 127.109 121.470314) (width 0.2) (layer "F.Cu") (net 4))
 (segment (start 129.090314 122.291) (end 127.929686 122.291) (width 0.2) (layer "F.Cu") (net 4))
 (segment (start 125.833 123.647) (end 125.833 103.363) (width 0.2) (layer "F.Cu") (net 6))
 (segment (start 125.833 103.363) (end 124.77 102.3) (width 0.2) (layer "F.Cu") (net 6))
 (segment (start 109.42 140.06) (end 125.833 123.647) (width 0.2) (layer "F.Cu") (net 6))
 (segment (start 128.46 140.02) (end 128.46 131.900686) (width 0.2) (layer "B.Cu") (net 7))
 (segment (start 116.310314 119.751) (end 115.149686 119.751) (width 0.2) (layer "B.Cu") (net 7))
 (segment (start 128.46 131.900686) (end 116.310314 119.751) (width 0.2) (layer "B.Cu") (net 7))
 (segment (start 114.329 118.930314) (end 114.329 115.281) (width 0.2) (layer "B.Cu") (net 7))
 (segment (start 114.329 115.281) (end 124.77 104.84) (width 0.2) (layer "B.Cu") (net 7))
 (segment (start 115.149686 119.751) (end 114.329 118.930314) (width 0.2) (layer "B.Cu") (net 7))
 (segment (start 108.019 125.21947) (end 114.329 118.90947) (width 0.2) (layer "F.Cu") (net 5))
 (segment (start 128.422314 137.761) (end 126.830421 139.352893) (width 0.2) (layer "F.Cu") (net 5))
 (segment (start 110.000314 141.461) (end 108.839686 141.461) (width 0.2) (layer "F.Cu") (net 5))
 (segment (start 108.839686 141.461) (end 108.019 140.640314) (width 0.2) (layer "F.Cu") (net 5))
 (segment (start 130.561314 139.9) (end 128.422314 137.761) (width 0.2) (layer "F.Cu") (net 5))
 (segment (start 147.52 139.9) (end 130.561314 139.9) (width 0.2) (layer "F.Cu") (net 5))
 (segment (start 108.019 140.640314) (end 108.019 125.21947) (width 0.2) (layer "F.Cu") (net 5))
 (segment (start 126.830421 139.352893) (end 112.108421 139.352893) (width 0.2) (layer "F.Cu") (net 5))
 (segment (start 114.329 118.90947) (end 114.329 116.74337) (width 0.2) (layer "F.Cu") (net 5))
 (segment (start 114.329 116.74337) (end 123.69237 107.38) (width 0.2) (layer "F.Cu") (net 5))
 (segment (start 123.69237 107.38) (end 124.77 107.38) (width 0.2) (layer "F.Cu") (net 5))
 (segment (start 112.108421 139.352893) (end 110.000314 141.461) (width 0.2) (layer "F.Cu") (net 5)))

